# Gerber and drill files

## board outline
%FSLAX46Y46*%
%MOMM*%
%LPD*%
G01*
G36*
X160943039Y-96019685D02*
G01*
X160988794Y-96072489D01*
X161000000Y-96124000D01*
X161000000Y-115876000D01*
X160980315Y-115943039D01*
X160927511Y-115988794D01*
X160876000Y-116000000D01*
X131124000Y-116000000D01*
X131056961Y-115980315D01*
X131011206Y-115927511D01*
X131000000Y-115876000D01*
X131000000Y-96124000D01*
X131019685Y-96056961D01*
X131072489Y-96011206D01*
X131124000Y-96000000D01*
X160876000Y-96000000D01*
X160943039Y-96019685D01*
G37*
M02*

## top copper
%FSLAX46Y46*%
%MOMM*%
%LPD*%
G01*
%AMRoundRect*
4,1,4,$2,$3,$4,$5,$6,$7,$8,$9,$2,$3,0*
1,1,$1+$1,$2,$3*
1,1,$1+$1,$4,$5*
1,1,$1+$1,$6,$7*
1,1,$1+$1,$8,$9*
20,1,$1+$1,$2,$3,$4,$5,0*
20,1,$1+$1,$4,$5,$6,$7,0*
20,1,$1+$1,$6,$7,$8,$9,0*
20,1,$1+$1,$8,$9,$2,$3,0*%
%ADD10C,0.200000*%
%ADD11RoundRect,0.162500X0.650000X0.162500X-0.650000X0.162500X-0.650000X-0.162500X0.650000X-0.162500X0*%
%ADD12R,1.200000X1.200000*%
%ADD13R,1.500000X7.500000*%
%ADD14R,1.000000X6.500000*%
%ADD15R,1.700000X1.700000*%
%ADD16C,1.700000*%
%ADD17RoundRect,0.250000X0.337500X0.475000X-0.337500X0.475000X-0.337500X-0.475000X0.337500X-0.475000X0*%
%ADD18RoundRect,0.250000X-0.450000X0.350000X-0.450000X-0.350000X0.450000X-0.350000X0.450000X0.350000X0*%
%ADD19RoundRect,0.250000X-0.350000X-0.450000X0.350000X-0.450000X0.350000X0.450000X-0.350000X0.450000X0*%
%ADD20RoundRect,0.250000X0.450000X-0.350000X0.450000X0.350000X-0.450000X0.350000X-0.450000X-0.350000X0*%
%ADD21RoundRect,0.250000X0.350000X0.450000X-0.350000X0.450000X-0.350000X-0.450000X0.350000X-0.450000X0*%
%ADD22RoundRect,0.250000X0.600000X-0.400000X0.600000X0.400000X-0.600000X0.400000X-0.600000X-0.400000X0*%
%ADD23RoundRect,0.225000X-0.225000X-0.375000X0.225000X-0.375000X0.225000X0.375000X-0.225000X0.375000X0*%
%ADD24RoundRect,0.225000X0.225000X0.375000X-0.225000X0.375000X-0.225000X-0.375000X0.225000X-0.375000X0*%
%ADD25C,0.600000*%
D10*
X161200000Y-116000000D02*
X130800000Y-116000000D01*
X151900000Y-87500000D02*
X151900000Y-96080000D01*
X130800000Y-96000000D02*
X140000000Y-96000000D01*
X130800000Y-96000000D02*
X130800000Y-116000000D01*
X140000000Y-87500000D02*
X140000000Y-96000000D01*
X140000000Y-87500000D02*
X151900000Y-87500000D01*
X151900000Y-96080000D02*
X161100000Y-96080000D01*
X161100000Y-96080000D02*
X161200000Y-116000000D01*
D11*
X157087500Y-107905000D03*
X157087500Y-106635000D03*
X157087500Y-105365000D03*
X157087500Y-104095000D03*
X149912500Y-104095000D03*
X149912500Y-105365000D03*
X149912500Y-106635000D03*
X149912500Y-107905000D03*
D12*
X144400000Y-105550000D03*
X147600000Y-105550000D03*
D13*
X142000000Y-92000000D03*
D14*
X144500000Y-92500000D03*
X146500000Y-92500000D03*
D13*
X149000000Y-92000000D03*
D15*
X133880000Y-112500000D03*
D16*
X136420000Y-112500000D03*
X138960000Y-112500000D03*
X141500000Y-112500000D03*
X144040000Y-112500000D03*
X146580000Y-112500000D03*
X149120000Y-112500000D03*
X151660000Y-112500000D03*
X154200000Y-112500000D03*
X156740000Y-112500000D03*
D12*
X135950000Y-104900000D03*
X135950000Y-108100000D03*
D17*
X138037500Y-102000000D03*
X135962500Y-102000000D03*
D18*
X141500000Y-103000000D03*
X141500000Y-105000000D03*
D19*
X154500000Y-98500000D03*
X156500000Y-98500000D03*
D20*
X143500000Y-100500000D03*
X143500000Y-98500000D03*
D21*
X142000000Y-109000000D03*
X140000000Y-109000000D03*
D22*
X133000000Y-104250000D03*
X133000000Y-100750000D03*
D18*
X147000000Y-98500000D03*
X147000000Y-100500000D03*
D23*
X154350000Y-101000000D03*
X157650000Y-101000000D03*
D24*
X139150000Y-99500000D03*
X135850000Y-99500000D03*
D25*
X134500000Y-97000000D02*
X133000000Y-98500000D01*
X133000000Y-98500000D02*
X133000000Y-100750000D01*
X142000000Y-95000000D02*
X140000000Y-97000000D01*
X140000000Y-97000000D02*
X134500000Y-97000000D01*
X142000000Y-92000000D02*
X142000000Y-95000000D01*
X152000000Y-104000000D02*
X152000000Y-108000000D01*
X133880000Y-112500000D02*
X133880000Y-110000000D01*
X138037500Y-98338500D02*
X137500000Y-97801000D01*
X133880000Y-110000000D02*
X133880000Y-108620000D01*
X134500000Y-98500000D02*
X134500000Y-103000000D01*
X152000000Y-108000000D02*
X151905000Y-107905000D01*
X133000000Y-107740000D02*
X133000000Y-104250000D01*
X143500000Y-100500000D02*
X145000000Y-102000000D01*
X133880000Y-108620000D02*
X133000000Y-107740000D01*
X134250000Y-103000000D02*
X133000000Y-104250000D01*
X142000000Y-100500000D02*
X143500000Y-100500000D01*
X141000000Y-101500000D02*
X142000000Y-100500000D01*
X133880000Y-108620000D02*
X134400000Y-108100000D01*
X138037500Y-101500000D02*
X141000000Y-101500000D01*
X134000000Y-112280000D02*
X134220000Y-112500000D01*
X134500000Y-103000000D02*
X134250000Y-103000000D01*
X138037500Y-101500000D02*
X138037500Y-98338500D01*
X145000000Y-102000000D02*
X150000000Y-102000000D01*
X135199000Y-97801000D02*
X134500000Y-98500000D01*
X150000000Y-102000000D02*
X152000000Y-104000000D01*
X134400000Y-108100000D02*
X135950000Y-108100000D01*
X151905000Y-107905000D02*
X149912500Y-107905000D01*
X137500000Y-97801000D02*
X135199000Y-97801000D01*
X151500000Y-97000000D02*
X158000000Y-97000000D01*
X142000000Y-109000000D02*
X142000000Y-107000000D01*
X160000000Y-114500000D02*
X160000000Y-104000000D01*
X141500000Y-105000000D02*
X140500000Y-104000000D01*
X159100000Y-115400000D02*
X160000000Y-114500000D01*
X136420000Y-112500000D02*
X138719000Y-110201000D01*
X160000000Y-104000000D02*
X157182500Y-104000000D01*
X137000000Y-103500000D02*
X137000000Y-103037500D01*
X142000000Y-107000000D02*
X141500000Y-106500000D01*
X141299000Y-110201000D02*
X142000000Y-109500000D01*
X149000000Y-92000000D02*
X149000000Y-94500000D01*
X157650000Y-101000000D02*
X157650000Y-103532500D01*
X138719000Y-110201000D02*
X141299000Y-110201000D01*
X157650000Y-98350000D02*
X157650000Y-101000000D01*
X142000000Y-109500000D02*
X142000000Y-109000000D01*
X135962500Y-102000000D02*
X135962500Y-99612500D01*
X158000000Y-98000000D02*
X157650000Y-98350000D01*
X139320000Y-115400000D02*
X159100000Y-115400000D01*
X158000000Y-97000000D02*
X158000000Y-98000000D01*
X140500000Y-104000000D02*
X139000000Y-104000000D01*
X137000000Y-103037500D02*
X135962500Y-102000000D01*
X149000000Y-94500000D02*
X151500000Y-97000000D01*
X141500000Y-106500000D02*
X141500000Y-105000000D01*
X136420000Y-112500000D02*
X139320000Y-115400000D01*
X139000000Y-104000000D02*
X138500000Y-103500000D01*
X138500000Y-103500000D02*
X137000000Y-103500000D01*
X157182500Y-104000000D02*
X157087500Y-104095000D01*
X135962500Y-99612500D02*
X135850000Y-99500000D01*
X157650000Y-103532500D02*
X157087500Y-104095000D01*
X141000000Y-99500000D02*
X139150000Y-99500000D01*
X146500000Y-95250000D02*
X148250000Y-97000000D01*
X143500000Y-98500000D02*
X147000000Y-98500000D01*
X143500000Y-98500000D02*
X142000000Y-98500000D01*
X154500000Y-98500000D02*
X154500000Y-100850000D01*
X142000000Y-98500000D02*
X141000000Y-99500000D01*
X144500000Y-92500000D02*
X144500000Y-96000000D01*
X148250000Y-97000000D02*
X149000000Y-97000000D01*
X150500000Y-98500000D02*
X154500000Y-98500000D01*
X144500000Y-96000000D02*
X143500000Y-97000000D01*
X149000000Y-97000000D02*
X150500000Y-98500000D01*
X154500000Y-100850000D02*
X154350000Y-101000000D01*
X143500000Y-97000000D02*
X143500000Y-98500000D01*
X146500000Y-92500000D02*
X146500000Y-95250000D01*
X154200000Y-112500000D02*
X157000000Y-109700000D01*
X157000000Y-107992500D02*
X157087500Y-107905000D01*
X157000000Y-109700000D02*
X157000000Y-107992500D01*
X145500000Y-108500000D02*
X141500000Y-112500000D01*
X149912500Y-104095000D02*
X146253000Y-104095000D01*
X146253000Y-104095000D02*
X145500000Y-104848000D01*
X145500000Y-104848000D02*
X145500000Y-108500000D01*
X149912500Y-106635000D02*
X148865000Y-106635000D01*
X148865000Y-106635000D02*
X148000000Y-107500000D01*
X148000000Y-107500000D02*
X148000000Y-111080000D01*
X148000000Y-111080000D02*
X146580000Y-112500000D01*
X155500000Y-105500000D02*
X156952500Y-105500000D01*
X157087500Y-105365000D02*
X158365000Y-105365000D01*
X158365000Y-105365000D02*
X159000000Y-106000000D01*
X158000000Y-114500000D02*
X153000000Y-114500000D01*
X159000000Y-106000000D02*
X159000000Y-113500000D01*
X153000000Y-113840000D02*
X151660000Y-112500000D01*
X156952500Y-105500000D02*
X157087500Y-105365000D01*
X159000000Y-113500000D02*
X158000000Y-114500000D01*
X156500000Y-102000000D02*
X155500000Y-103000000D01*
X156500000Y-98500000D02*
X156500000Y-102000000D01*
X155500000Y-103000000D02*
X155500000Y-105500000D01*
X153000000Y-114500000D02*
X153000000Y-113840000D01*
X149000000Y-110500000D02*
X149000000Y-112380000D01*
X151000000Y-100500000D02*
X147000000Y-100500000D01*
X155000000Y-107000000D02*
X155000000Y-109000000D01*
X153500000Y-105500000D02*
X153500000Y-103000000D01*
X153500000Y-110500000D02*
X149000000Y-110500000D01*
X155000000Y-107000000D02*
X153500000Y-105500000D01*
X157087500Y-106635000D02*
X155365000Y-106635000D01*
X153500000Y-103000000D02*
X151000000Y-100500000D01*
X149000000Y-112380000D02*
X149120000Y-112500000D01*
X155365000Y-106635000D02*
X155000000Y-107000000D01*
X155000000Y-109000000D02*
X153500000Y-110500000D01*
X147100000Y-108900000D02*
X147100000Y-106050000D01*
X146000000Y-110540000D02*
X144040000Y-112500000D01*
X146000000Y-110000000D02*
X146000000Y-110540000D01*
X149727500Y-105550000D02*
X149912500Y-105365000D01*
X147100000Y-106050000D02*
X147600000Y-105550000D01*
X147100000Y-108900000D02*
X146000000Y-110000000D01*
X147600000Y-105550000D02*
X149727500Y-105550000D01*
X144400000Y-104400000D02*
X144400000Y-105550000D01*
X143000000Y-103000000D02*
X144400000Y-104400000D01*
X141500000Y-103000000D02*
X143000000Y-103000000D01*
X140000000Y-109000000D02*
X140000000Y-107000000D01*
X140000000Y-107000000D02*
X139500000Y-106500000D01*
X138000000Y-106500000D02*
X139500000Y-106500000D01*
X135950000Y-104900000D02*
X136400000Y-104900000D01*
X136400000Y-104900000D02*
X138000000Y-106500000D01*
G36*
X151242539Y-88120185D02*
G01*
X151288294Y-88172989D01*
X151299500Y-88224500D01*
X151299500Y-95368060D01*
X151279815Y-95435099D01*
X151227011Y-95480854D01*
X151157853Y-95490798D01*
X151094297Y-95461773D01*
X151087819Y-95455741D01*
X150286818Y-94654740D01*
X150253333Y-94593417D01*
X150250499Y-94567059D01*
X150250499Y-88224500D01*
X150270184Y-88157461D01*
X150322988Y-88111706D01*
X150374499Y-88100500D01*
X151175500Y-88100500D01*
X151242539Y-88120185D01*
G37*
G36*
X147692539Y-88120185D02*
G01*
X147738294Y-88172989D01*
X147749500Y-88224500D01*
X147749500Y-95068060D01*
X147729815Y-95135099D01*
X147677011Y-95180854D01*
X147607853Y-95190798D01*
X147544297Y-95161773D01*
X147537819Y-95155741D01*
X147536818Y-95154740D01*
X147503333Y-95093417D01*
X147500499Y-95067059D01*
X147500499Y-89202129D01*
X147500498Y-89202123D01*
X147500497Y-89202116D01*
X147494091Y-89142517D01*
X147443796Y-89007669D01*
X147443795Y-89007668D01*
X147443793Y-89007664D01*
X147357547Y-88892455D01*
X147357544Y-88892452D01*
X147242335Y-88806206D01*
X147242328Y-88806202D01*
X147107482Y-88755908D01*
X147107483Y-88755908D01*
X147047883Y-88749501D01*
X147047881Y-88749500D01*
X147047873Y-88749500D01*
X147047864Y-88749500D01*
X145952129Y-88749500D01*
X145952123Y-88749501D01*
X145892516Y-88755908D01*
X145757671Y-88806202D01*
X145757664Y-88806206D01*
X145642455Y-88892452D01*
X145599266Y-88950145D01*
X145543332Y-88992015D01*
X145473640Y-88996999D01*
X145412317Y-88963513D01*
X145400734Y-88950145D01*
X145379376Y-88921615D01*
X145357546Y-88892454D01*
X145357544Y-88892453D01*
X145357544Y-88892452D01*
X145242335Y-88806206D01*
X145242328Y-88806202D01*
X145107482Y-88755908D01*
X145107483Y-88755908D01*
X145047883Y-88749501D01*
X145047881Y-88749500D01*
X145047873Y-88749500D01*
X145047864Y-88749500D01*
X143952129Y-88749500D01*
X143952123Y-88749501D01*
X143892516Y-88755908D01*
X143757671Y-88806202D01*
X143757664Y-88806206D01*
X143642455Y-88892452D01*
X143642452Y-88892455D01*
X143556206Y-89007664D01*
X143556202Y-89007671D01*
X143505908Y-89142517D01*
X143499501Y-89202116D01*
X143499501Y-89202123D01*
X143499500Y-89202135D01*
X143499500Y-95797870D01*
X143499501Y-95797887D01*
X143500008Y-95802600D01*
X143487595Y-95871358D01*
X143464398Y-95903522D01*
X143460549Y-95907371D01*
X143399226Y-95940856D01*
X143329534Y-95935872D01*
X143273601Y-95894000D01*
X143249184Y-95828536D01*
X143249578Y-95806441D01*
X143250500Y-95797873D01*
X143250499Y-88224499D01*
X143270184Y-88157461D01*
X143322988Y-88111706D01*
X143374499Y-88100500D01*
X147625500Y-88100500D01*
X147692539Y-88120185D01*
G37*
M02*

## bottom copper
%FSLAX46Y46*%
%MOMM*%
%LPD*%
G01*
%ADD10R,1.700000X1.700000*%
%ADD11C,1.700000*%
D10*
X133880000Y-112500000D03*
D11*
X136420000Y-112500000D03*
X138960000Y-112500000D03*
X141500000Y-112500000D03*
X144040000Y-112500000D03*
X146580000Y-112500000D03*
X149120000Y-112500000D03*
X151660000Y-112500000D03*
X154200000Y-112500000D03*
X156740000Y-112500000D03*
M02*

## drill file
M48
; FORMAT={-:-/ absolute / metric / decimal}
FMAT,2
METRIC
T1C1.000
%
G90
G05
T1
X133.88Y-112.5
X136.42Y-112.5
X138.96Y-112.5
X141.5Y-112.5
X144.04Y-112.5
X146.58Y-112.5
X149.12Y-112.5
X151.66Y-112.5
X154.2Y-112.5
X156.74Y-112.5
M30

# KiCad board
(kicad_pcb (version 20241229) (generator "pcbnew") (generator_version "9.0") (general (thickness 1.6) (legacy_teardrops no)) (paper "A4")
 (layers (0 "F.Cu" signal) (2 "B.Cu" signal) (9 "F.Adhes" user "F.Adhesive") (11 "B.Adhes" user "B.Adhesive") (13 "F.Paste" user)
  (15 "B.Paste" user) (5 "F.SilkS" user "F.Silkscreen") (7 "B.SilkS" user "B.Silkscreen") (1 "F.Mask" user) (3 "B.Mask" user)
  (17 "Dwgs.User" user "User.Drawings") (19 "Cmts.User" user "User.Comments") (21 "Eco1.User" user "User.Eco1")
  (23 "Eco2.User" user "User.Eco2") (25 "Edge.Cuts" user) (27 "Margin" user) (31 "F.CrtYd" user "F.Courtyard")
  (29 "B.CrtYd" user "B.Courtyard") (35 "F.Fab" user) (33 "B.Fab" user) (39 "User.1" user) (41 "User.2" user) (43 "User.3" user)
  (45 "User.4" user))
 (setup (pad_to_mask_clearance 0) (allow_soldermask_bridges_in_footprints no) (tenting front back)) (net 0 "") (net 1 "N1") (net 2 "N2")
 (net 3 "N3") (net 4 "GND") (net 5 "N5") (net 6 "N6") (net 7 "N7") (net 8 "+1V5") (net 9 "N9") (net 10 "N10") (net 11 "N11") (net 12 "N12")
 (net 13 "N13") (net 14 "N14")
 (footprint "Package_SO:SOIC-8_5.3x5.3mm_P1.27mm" (layer "F.Cu") (at 153.5 106 180)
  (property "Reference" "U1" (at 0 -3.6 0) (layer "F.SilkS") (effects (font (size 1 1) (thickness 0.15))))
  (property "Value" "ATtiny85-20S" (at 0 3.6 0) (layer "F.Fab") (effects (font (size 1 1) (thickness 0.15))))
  (pad "1" smd roundrect (at -3.5875 -1.905 180) (size 1.625 0.65) (layers "F.Cu" "F.Mask" "F.Paste") (roundrect_rratio 0.25) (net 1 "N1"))
  (pad "2" smd roundrect (at -3.5875 -0.635 180) (size 1.625 0.65) (layers "F.Cu" "F.Mask" "F.Paste") (roundrect_rratio 0.25) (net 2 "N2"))
  (pad "3" smd roundrect (at -3.5875 0.635 180) (size 1.625 0.65) (layers "F.Cu" "F.Mask" "F.Paste") (roundrect_rratio 0.25) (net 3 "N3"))
  (pad "4" smd roundrect (at -3.5875 1.905 180) (size 1.625 0.65) (layers "F.Cu" "F.Mask" "F.Paste") (roundrect_rratio 0.25) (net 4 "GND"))
  (pad "5" smd roundrect (at 3.5875 1.905 180) (size 1.625 0.65) (layers "F.Cu" "F.Mask" "F.Paste") (roundrect_rratio 0.25) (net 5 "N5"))
  (pad "6" smd roundrect (at 3.5875 0.635 180) (size 1.625 0.65) (layers "F.Cu" "F.Mask" "F.Paste") (roundrect_rratio 0.25) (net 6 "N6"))
  (pad "7" smd roundrect (at 3.5875 -0.635 180) (size 1.625 0.65) (layers "F.Cu" "F.Mask" "F.Paste") (roundrect_rratio 0.25) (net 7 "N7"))
  (pad "8" smd roundrect (at 3.5875 -1.905 180) (size 1.625 0.65) (layers "F.Cu" "F.Mask" "F.Paste") (roundrect_rratio 0.25) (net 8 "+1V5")))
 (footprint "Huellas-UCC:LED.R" (layer "F.Cu") (at 146.5 105.1)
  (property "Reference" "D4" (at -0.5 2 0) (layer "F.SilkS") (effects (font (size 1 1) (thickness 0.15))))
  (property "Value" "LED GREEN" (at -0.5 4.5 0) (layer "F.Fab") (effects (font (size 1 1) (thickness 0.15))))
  (pad "1" smd rect (at -2.1 0.45) (size 1.2 1.2) (layers "F.Cu" "F.Mask" "F.Paste") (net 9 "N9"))
  (pad "2" smd rect (at 1.1 0.45) (size 1.2 1.2) (layers "F.Cu" "F.Mask" "F.Paste") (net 6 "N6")))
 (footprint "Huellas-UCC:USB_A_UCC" (layer "F.Cu") (at 145.5 92.2 -90)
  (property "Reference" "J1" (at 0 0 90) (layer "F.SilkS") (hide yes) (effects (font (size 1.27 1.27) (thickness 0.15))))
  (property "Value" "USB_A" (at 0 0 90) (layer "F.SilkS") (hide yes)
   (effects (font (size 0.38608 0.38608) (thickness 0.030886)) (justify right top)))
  (pad "1" smd rect (at -0.2 3.5 270) (size 7.5 1.5) (layers "F.Cu" "F.Mask" "F.Paste") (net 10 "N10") (solder_mask_margin 0.1016))
  (pad "2" smd rect (at 0.3 1 270) (size 6.5 1) (layers "F.Cu" "F.Mask" "F.Paste") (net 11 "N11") (solder_mask_margin 0.1016))
  (pad "3" smd rect (at 0.3 -1 270) (size 6.5 1) (layers "F.Cu" "F.Mask" "F.Paste") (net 11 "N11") (solder_mask_margin 0.1016))
  (pad "4" smd rect (at -0.2 -3.5 270) (size 7.5 1.5) (layers "F.Cu" "F.Mask" "F.Paste") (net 4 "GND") (solder_mask_margin 0.1016)))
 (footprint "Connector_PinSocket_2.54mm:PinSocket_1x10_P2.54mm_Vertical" (layer "F.Cu") (at 133.88 112.5 90)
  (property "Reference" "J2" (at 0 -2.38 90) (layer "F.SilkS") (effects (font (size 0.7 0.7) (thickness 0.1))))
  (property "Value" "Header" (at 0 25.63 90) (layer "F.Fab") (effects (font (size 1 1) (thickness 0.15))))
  (pad "1" thru_hole rect (at 0 0 90) (size 1.7 1.7) (drill 1) (layers "*.Cu" "*.Mask") (remove_unused_layers no) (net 8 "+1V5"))
  (pad "2" thru_hole circle (at 0 2.54 90) (size 1.7 1.7) (drill 1) (layers "*.Cu" "*.Mask") (remove_unused_layers no) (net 4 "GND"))
  (pad "3" thru_hole circle (at 0 5.08 90) (size 1.7 1.7) (drill 1) (layers "*.Cu" "*.Mask") (remove_unused_layers no) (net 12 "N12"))
  (pad "4" thru_hole circle (at 0 7.62 90) (size 1.7 1.7) (drill 1) (layers "*.Cu" "*.Mask") (remove_unused_layers no) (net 5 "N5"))
  (pad "5" thru_hole circle (at 0 10.16 90) (size 1.7 1.7) (drill 1) (layers "*.Cu" "*.Mask") (remove_unused_layers no) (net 6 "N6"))
  (pad "6" thru_hole circle (at 0 12.7 90) (size 1.7 1.7) (drill 1) (layers "*.Cu" "*.Mask") (remove_unused_layers no) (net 7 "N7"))
  (pad "7" thru_hole circle (at 0 15.24 90) (size 1.7 1.7) (drill 1) (layers "*.Cu" "*.Mask") (remove_unused_layers no) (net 2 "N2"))
  (pad "8" thru_hole circle (at 0 17.78 90) (size 1.7 1.7) (drill 1) (layers "*.Cu" "*.Mask") (remove_unused_layers no) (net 3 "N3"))
  (pad "9" thru_hole circle (at 0 20.32 90) (size 1.7 1.7) (drill 1) (layers "*.Cu" "*.Mask") (remove_unused_layers no) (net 1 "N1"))
  (pad "10" thru_hole circle (at 0 22.86 90) (size 1.7 1.7) (drill 1) (layers "*.Cu" "*.Mask") (remove_unused_layers no) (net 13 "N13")))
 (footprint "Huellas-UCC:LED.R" (layer "F.Cu") (at 136.4 107 -90)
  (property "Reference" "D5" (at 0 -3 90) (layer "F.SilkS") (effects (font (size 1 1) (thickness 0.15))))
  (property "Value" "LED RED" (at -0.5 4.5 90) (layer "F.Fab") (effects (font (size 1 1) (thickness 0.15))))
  (pad "1" smd rect (at -2.1 0.45 270) (size 1.2 1.2) (layers "F.Cu" "F.Mask" "F.Paste") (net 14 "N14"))
  (pad "2" smd rect (at 1.1 0.45 270) (size 1.2 1.2) (layers "F.Cu" "F.Mask" "F.Paste") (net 8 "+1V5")))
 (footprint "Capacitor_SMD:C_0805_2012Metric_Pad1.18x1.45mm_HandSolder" (layer "F.Cu") (at 137 102 180)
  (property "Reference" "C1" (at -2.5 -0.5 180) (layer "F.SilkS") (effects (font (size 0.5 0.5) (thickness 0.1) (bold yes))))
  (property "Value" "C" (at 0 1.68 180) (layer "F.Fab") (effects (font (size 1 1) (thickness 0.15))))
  (pad "1" smd roundrect (at -1.0375 0 180) (size 1.175 1.45) (layers "F.Cu" "F.Mask" "F.Paste") (roundrect_rratio 0.212766) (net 8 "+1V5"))
  (pad "2" smd roundrect (at 1.0375 0 180) (size 1.175 1.45) (layers "F.Cu" "F.Mask" "F.Paste") (roundrect_rratio 0.212766) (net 4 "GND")))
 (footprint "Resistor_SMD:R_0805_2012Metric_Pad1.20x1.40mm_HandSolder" (layer "F.Cu") (at 141.5 104 -90)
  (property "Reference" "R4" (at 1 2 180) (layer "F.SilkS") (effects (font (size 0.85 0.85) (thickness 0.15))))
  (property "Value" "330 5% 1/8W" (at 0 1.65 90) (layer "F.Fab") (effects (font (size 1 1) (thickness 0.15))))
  (pad "1" smd roundrect (at -1 0 270) (size 1.2 1.4) (layers "F.Cu" "F.Mask" "F.Paste") (roundrect_rratio 0.208333) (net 9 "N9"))
  (pad "2" smd roundrect (at 1 0 270) (size 1.2 1.4) (layers "F.Cu" "F.Mask" "F.Paste") (roundrect_rratio 0.208333) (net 4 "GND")))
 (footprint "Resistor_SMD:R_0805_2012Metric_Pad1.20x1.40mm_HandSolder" (layer "F.Cu") (at 155.5 98.5)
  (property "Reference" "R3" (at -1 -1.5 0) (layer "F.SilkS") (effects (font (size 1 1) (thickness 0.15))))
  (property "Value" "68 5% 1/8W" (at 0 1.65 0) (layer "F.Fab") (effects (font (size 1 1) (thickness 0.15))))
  (pad "1" smd roundrect (at -1 0) (size 1.2 1.4) (layers "F.Cu" "F.Mask" "F.Paste") (roundrect_rratio 0.208333) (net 11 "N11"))
  (pad "2" smd roundrect (at 1 0) (size 1.2 1.4) (layers "F.Cu" "F.Mask" "F.Paste") (roundrect_rratio 0.208333) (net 3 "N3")))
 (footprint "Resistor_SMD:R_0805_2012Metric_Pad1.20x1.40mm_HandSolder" (layer "F.Cu") (at 143.5 99.5 90)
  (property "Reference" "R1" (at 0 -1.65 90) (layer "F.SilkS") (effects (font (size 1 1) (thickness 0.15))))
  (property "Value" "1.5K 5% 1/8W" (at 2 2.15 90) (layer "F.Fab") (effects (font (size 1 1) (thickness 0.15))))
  (pad "1" smd roundrect (at -1 0 90) (size 1.2 1.4) (layers "F.Cu" "F.Mask" "F.Paste") (roundrect_rratio 0.208333) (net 8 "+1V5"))
  (pad "2" smd roundrect (at 1 0 90) (size 1.2 1.4) (layers "F.Cu" "F.Mask" "F.Paste") (roundrect_rratio 0.208333) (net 11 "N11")))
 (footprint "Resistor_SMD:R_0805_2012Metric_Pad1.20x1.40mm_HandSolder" (layer "F.Cu") (at 141 109 180)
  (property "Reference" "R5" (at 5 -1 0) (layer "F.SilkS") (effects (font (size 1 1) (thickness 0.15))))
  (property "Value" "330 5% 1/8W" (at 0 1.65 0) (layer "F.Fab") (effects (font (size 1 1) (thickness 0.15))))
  (pad "1" smd roundrect (at -1 0 180) (size 1.2 1.4) (layers "F.Cu" "F.Mask" "F.Paste") (roundrect_rratio 0.208333) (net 4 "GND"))
  (pad "2" smd roundrect (at 1 0 180) (size 1.2 1.4) (layers "F.Cu" "F.Mask" "F.Paste") (roundrect_rratio 0.208333) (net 14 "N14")))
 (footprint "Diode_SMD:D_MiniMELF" (layer "F.Cu") (at 133 102.5 90)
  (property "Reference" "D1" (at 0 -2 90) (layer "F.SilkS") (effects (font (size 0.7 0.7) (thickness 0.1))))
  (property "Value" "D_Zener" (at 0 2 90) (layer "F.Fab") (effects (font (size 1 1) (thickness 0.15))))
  (pad "1" smd roundrect (at -1.75 0 90) (size 1.3 1.7) (layers "F.Cu" "F.Mask" "F.Paste") (roundrect_rratio 0.1923076923) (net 8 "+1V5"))
  (pad "2" smd roundrect (at 1.75 0 90) (size 1.3 1.7) (layers "F.Cu" "F.Mask" "F.Paste") (roundrect_rratio 0.1923076923) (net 10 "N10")))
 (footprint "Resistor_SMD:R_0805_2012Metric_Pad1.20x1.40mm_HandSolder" (layer "F.Cu") (at 147 99.5 -90)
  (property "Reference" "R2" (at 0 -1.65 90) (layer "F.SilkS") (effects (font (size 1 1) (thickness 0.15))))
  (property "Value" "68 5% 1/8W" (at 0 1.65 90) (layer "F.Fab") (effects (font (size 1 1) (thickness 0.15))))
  (pad "1" smd roundrect (at -1 0 270) (size 1.2 1.4) (layers "F.Cu" "F.Mask" "F.Paste") (roundrect_rratio 0.208333) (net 11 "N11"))
  (pad "2" smd roundrect (at 1 0 270) (size 1.2 1.4) (layers "F.Cu" "F.Mask" "F.Paste") (roundrect_rratio 0.208333) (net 2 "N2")))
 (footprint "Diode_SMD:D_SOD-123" (layer "F.Cu") (at 156 101)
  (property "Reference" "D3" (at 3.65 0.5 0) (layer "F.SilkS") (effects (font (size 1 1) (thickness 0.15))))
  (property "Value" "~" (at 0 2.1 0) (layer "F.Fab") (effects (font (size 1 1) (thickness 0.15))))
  (pad "1" smd roundrect (at -1.65 0) (size 0.9 1.2) (layers "F.Cu" "F.Mask" "F.Paste") (roundrect_rratio 0.25) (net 11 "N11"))
  (pad "2" smd roundrect (at 1.65 0) (size 0.9 1.2) (layers "F.Cu" "F.Mask" "F.Paste") (roundrect_rratio 0.25) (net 4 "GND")))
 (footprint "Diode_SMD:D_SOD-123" (layer "F.Cu") (at 137.5 99.5 180)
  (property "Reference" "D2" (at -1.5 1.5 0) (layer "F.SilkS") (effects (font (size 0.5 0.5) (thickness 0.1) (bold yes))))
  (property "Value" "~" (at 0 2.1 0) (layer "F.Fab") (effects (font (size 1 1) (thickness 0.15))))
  (pad "1" smd roundrect (at -1.65 0 180) (size 0.9 1.2) (layers "F.Cu" "F.Mask" "F.Paste") (roundrect_rratio 0.25) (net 11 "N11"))
  (pad "2" smd roundrect (at 1.65 0 180) (size 0.9 1.2) (layers "F.Cu" "F.Mask" "F.Paste") (roundrect_rratio 0.25) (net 4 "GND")))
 (gr_line (start 161.2 116) (end 130.8 116) (stroke (width 0.2) (type solid)) (layer "F.Cu"))
 (gr_line (start 151.9 87.5) (end 151.9 96.08) (stroke (width 0.2) (type solid)) (layer "F.Cu"))
 (gr_line (start 130.8 96) (end 140 96) (stroke (width 0.2) (type solid)) (layer "F.Cu"))
 (gr_line (start 130.8 96) (end 130.8 116) (stroke (width 0.2) (type solid)) (layer "F.Cu"))
 (gr_line (start 140 87.5) (end 140 96) (stroke (width 0.2) (type solid)) (layer "F.Cu"))
 (gr_line (start 140 87.5) (end 151.9 87.5) (stroke (width 0.2) (type default)) (layer "F.Cu"))
 (gr_line (start 151.9 96.08) (end 161.1 96.08) (stroke (width 0.2) (type solid)) (layer "F.Cu"))
 (gr_line (start 161.1 96.08) (end 161.2 116) (stroke (width 0.2) (type solid)) (layer "F.Cu"))
 (segment (start 134.5 97) (end 133 98.5) (width 0.6) (layer "F.Cu") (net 10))
 (segment (start 133 98.5) (end 133 100.75) (width 0.6) (layer "F.Cu") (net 10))
 (segment (start 142 95) (end 140 97) (width 0.6) (layer "F.Cu") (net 10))
 (segment (start 140 97) (end 134.5 97) (width 0.6) (layer "F.Cu") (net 10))
 (segment (start 142 92) (end 142 95) (width 0.6) (layer "F.Cu") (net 10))
 (segment (start 152 104) (end 152 108) (width 0.6) (layer "F.Cu") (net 8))
 (segment (start 133.88 112.5) (end 133.88 110) (width 0.6) (layer "F.Cu") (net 8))
 (segment (start 138.0375 98.3385) (end 137.5 97.801) (width 0.6) (layer "F.Cu") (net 8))
 (segment (start 133.88 110) (end 133.88 108.62) (width 0.6) (layer "F.Cu") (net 8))
 (segment (start 134.5 98.5) (end 134.5 103) (width 0.6) (layer "F.Cu") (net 8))
 (segment (start 152 108) (end 151.905 107.905) (width 0.6) (layer "F.Cu") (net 8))
 (segment (start 133 107.74) (end 133 104.25) (width 0.6) (layer "F.Cu") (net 8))
 (segment (start 143.5 100.5) (end 145 102) (width 0.6) (layer "F.Cu") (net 8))
 (segment (start 133.88 108.62) (end 133 107.74) (width 0.6) (layer "F.Cu") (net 8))
 (segment (start 134.25 103) (end 133 104.25) (width 0.6) (layer "F.Cu") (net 8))
 (segment (start 142 100.5) (end 143.5 100.5) (width 0.6) (layer "F.Cu") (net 8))
 (segment (start 141 101.5) (end 142 100.5) (width 0.6) (layer "F.Cu") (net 8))
 (segment (start 133.88 108.62) (end 134.4 108.1) (width 0.6) (layer "F.Cu") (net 8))
 (segment (start 138.0375 101.5) (end 141 101.5) (width 0.6) (layer "F.Cu") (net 8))
 (segment (start 134 112.28) (end 134.22 112.5) (width 0.6) (layer "F.Cu") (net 8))
 (segment (start 134.5 103) (end 134.25 103) (width 0.6) (layer "F.Cu") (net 8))
 (segment (start 138.0375 101.5) (end 138.0375 98.3385) (width 0.6) (layer "F.Cu") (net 8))
 (segment (start 145 102) (end 150 102) (width 0.6) (layer "F.Cu") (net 8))
 (segment (start 135.199 97.801) (end 134.5 98.5) (width 0.6) (layer "F.Cu") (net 8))
 (segment (start 150 102) (end 152 104) (width 0.6) (layer "F.Cu") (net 8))
 (segment (start 134.4 108.1) (end 135.95 108.1) (width 0.6) (layer "F.Cu") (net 8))
 (segment (start 151.905 107.905) (end 149.9125 107.905) (width 0.6) (layer "F.Cu") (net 8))
 (segment (start 137.5 97.801) (end 135.199 97.801) (width 0.6) (layer "F.Cu") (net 8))
 (segment (start 151.5 97) (end 158 97) (width 0.6) (layer "F.Cu") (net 4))
 (segment (start 142 109) (end 142 107) (width 0.6) (layer "F.Cu") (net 4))
 (segment (start 160 114.5) (end 160 104) (width 0.6) (layer "F.Cu") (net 4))
 (segment (start 141.5 105) (end 140.5 104) (width 0.6) (layer "F.Cu") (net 4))
 (segment (start 159.1 115.4) (end 160 114.5) (width 0.6) (layer "F.Cu") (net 4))
 (segment (start 136.42 112.5) (end 138.719 110.201) (width 0.6) (layer "F.Cu") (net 4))
 (segment (start 160 104) (end 157.1825 104) (width 0.6) (layer "F.Cu") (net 4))
 (segment (start 137 103.5) (end 137 103.0375) (width 0.6) (layer "F.Cu") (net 4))
 (segment (start 142 107) (end 141.5 106.5) (width 0.6) (layer "F.Cu") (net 4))
 (segment (start 141.299 110.201) (end 142 109.5) (width 0.6) (layer "F.Cu") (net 4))
 (segment (start 149 92) (end 149 94.5) (width 0.6) (layer "F.Cu") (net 4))
 (segment (start 157.65 101) (end 157.65 103.5325) (width 0.6) (layer "F.Cu") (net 4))
 (segment (start 138.719 110.201) (end 141.299 110.201) (width 0.6) (layer "F.Cu") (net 4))
 (segment (start 157.65 98.35) (end 157.65 101) (width 0.6) (layer "F.Cu") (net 4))
 (segment (start 142 109.5) (end 142 109) (width 0.6) (layer "F.Cu") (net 4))
 (segment (start 135.9625 102) (end 135.9625 99.6125) (width 0.6) (layer "F.Cu") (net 4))
 (segment (start 158 98) (end 157.65 98.35) (width 0.6) (layer "F.Cu") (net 4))
 (segment (start 139.32 115.4) (end 159.1 115.4) (width 0.6) (layer "F.Cu") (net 4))
 (segment (start 158 97) (end 158 98) (width 0.6) (layer "F.Cu") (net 4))
 (segment (start 140.5 104) (end 139 104) (width 0.6) (layer "F.Cu") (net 4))
 (segment (start 137 103.0375) (end 135.9625 102) (width 0.6) (layer "F.Cu") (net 4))
 (segment (start 149 94.5) (end 151.5 97) (width 0.6) (layer "F.Cu") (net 4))
 (segment (start 141.5 106.5) (end 141.5 105) (width 0.6) (layer "F.Cu") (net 4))
 (segment (start 136.42 112.5) (end 139.32 115.4) (width 0.6) (layer "F.Cu") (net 4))
 (segment (start 139 104) (end 138.5 103.5) (width 0.6) (layer "F.Cu") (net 4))
 (segment (start 138.5 103.5) (end 137 103.5) (width 0.6) (layer "F.Cu") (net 4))
 (segment (start 157.1825 104) (end 157.0875 104.095) (width 0.6) (layer "F.Cu") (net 4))
 (segment (start 135.9625 99.6125) (end 135.85 99.5) (width 0.6) (layer "F.Cu") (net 4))
 (segment (start 157.65 103.5325) (end 157.0875 104.095) (width 0.6) (layer "F.Cu") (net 4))
 (segment (start 141 99.5) (end 139.15 99.5) (width 0.6) (layer "F.Cu") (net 11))
 (segment (start 146.5 95.25) (end 148.25 97) (width 0.6) (layer "F.Cu") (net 11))
 (segment (start 143.5 98.5) (end 147 98.5) (width 0.6) (layer "F.Cu") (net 11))
 (segment (start 143.5 98.5) (end 142 98.5) (width 0.6) (layer "F.Cu") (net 11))
 (segment (start 154.5 98.5) (end 154.5 100.85) (width 0.6) (layer "F.Cu") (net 11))
 (segment (start 142 98.5) (end 141 99.5) (width 0.6) (layer "F.Cu") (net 11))
 (segment (start 144.5 92.5) (end 144.5 96) (width 0.6) (layer "F.Cu") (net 11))
 (segment (start 148.25 97) (end 149 97) (width 0.6) (layer "F.Cu") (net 11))
 (segment (start 150.5 98.5) (end 154.5 98.5) (width 0.6) (layer "F.Cu") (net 11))
 (segment (start 144.5 96) (end 143.5 97) (width 0.6) (layer "F.Cu") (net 11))
 (segment (start 149 97) (end 150.5 98.5) (width 0.6) (layer "F.Cu") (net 11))
 (segment (start 154.5 100.85) (end 154.35 101) (width 0.6) (layer "F.Cu") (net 11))
 (segment (start 143.5 97) (end 143.5 98.5) (width 0.6) (layer "F.Cu") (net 11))
 (segment (start 146.5 92.5) (end 146.5 95.25) (width 0.6) (layer "F.Cu") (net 11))
 (segment (start 154.2 112.5) (end 157 109.7) (width 0.6) (layer "F.Cu") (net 1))
 (segment (start 157 107.9925) (end 157.0875 107.905) (width 0.6) (layer "F.Cu") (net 1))
 (segment (start 157 109.7) (end 157 107.9925) (width 0.6) (layer "F.Cu") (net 1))
 (segment (start 145.5 108.5) (end 141.5 112.5) (width 0.6) (layer "F.Cu") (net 5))
 (segment (start 149.9125 104.095) (end 146.253 104.095) (width 0.6) (layer "F.Cu") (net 5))
 (segment (start 146.253 104.095) (end 145.5 104.848) (width 0.6) (layer "F.Cu") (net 5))
 (segment (start 145.5 104.848) (end 145.5 108.5) (width 0.6) (layer "F.Cu") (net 5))
 (segment (start 149.9125 106.635) (end 148.865 106.635) (width 0.6) (layer "F.Cu") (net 7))
 (segment (start 148.865 106.635) (end 148 107.5) (width 0.6) (layer "F.Cu") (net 7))
 (segment (start 148 107.5) (end 148 111.08) (width 0.6) (layer "F.Cu") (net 7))
 (segment (start 148 111.08) (end 146.58 112.5) (width 0.6) (layer "F.Cu") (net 7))
 (segment (start 155.5 105.5) (end 156.9525 105.5) (width 0.6) (layer "F.Cu") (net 3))
 (segment (start 157.0875 105.365) (end 158.365 105.365) (width 0.6) (layer "F.Cu") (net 3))
 (segment (start 158.365 105.365) (end 159 106) (width 0.6) (layer "F.Cu") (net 3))
 (segment (start 158 114.5) (end 153 114.5) (width 0.6) (layer "F.Cu") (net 3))
 (segment (start 159 106) (end 159 113.5) (width 0.6) (layer "F.Cu") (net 3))
 (segment (start 153 113.84) (end 151.66 112.5) (width 0.6) (layer "F.Cu") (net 3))
 (segment (start 156.9525 105.5) (end 157.0875 105.365) (width 0.6) (layer "F.Cu") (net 3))
 (segment (start 159 113.5) (end 158 114.5) (width 0.6) (layer "F.Cu") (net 3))
 (segment (start 156.5 102) (end 155.5 103) (width 0.6) (layer "F.Cu") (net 3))
 (segment (start 156.5 98.5) (end 156.5 102) (width 0.6) (layer "F.Cu") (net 3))
 (segment (start 155.5 103) (end 155.5 105.5) (width 0.6) (layer "F.Cu") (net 3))
 (segment (start 153 114.5) (end 153 113.84) (width 0.6) (layer "F.Cu") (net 3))
 (segment (start 149 110.5) (end 149 112.38) (width 0.6) (layer "F.Cu") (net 2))
 (segment (start 151 100.5) (end 147 100.5) (width 0.6) (layer "F.Cu") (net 2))
 (segment (start 155 107) (end 155 109) (width 0.6) (layer "F.Cu") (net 2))
 (segment (start 153.5 105.5) (end 153.5 103) (width 0.6) (layer "F.Cu") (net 2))
 (segment (start 153.5 110.5) (end 149 110.5) (width 0.6) (layer "F.Cu") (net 2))
 (segment (start 155 107) (end 153.5 105.5) (width 0.6) (layer "F.Cu") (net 2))
 (segment (start 157.0875 106.635) (end 155.365 106.635) (width 0.6) (layer "F.Cu") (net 2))
 (segment (start 153.5 103) (end 151 100.5) (width 0.6) (layer "F.Cu") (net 2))
 (segment (start 149 112.38) (end 149.12 112.5) (width 0.6) (layer "F.Cu") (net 2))
 (segment (start 155.365 106.635) (end 155 107) (width 0.6) (layer "F.Cu") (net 2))
 (segment (start 155 109) (end 153.5 110.5) (width 0.6) (layer "F.Cu") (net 2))
 (segment (start 147.1 108.9) (end 147.1 106.05) (width 0.6) (layer "F.Cu") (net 6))
 (segment (start 146 110.54) (end 144.04 112.5) (width 0.6) (layer "F.Cu") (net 6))
 (segment (start 146 110) (end 146 110.54) (width 0.6) (layer "F.Cu") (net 6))
 (segment (start 149.7275 105.55) (end 149.9125 105.365) (width 0.6) (layer "F.Cu") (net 6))
 (segment (start 147.1 106.05) (end 147.6 105.55) (width 0.6) (layer "F.Cu") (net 6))
 (segment (start 147.1 108.9) (end 146 110) (width 0.6) (layer "F.Cu") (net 6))
 (segment (start 147.6 105.55) (end 149.7275 105.55) (width 0.6) (layer "F.Cu") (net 6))
 (segment (start 144.4 104.4) (end 144.4 105.55) (width 0.6) (layer "F.Cu") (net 9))
 (segment (start 143 103) (end 144.4 104.4) (width 0.6) (layer "F.Cu") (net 9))
 (segment (start 141.5 103) (end 143 103) (width 0.6) (layer "F.Cu") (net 9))
 (segment (start 140 109) (end 140 107) (width 0.6) (layer "F.Cu") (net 14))
 (segment (start 140 107) (end 139.5 106.5) (width 0.6) (layer "F.Cu") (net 14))
 (segment (start 138 106.5) (end 139.5 106.5) (width 0.6) (layer "F.Cu") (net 14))
 (segment (start 135.95 104.9) (end 136.4 104.9) (width 0.6) (layer "F.Cu") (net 14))
 (segment (start 136.4 104.9) (end 138 106.5) (width 0.6) (layer "F.Cu") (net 14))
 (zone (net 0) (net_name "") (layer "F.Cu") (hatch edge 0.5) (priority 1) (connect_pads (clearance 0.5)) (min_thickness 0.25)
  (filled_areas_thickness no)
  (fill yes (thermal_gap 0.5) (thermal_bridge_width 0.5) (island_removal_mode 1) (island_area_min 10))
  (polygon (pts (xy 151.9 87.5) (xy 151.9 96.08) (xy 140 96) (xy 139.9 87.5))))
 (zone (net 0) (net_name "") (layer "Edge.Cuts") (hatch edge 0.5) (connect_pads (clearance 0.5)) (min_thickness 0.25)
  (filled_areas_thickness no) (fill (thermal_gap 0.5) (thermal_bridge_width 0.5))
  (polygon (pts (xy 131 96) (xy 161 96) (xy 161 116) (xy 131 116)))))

